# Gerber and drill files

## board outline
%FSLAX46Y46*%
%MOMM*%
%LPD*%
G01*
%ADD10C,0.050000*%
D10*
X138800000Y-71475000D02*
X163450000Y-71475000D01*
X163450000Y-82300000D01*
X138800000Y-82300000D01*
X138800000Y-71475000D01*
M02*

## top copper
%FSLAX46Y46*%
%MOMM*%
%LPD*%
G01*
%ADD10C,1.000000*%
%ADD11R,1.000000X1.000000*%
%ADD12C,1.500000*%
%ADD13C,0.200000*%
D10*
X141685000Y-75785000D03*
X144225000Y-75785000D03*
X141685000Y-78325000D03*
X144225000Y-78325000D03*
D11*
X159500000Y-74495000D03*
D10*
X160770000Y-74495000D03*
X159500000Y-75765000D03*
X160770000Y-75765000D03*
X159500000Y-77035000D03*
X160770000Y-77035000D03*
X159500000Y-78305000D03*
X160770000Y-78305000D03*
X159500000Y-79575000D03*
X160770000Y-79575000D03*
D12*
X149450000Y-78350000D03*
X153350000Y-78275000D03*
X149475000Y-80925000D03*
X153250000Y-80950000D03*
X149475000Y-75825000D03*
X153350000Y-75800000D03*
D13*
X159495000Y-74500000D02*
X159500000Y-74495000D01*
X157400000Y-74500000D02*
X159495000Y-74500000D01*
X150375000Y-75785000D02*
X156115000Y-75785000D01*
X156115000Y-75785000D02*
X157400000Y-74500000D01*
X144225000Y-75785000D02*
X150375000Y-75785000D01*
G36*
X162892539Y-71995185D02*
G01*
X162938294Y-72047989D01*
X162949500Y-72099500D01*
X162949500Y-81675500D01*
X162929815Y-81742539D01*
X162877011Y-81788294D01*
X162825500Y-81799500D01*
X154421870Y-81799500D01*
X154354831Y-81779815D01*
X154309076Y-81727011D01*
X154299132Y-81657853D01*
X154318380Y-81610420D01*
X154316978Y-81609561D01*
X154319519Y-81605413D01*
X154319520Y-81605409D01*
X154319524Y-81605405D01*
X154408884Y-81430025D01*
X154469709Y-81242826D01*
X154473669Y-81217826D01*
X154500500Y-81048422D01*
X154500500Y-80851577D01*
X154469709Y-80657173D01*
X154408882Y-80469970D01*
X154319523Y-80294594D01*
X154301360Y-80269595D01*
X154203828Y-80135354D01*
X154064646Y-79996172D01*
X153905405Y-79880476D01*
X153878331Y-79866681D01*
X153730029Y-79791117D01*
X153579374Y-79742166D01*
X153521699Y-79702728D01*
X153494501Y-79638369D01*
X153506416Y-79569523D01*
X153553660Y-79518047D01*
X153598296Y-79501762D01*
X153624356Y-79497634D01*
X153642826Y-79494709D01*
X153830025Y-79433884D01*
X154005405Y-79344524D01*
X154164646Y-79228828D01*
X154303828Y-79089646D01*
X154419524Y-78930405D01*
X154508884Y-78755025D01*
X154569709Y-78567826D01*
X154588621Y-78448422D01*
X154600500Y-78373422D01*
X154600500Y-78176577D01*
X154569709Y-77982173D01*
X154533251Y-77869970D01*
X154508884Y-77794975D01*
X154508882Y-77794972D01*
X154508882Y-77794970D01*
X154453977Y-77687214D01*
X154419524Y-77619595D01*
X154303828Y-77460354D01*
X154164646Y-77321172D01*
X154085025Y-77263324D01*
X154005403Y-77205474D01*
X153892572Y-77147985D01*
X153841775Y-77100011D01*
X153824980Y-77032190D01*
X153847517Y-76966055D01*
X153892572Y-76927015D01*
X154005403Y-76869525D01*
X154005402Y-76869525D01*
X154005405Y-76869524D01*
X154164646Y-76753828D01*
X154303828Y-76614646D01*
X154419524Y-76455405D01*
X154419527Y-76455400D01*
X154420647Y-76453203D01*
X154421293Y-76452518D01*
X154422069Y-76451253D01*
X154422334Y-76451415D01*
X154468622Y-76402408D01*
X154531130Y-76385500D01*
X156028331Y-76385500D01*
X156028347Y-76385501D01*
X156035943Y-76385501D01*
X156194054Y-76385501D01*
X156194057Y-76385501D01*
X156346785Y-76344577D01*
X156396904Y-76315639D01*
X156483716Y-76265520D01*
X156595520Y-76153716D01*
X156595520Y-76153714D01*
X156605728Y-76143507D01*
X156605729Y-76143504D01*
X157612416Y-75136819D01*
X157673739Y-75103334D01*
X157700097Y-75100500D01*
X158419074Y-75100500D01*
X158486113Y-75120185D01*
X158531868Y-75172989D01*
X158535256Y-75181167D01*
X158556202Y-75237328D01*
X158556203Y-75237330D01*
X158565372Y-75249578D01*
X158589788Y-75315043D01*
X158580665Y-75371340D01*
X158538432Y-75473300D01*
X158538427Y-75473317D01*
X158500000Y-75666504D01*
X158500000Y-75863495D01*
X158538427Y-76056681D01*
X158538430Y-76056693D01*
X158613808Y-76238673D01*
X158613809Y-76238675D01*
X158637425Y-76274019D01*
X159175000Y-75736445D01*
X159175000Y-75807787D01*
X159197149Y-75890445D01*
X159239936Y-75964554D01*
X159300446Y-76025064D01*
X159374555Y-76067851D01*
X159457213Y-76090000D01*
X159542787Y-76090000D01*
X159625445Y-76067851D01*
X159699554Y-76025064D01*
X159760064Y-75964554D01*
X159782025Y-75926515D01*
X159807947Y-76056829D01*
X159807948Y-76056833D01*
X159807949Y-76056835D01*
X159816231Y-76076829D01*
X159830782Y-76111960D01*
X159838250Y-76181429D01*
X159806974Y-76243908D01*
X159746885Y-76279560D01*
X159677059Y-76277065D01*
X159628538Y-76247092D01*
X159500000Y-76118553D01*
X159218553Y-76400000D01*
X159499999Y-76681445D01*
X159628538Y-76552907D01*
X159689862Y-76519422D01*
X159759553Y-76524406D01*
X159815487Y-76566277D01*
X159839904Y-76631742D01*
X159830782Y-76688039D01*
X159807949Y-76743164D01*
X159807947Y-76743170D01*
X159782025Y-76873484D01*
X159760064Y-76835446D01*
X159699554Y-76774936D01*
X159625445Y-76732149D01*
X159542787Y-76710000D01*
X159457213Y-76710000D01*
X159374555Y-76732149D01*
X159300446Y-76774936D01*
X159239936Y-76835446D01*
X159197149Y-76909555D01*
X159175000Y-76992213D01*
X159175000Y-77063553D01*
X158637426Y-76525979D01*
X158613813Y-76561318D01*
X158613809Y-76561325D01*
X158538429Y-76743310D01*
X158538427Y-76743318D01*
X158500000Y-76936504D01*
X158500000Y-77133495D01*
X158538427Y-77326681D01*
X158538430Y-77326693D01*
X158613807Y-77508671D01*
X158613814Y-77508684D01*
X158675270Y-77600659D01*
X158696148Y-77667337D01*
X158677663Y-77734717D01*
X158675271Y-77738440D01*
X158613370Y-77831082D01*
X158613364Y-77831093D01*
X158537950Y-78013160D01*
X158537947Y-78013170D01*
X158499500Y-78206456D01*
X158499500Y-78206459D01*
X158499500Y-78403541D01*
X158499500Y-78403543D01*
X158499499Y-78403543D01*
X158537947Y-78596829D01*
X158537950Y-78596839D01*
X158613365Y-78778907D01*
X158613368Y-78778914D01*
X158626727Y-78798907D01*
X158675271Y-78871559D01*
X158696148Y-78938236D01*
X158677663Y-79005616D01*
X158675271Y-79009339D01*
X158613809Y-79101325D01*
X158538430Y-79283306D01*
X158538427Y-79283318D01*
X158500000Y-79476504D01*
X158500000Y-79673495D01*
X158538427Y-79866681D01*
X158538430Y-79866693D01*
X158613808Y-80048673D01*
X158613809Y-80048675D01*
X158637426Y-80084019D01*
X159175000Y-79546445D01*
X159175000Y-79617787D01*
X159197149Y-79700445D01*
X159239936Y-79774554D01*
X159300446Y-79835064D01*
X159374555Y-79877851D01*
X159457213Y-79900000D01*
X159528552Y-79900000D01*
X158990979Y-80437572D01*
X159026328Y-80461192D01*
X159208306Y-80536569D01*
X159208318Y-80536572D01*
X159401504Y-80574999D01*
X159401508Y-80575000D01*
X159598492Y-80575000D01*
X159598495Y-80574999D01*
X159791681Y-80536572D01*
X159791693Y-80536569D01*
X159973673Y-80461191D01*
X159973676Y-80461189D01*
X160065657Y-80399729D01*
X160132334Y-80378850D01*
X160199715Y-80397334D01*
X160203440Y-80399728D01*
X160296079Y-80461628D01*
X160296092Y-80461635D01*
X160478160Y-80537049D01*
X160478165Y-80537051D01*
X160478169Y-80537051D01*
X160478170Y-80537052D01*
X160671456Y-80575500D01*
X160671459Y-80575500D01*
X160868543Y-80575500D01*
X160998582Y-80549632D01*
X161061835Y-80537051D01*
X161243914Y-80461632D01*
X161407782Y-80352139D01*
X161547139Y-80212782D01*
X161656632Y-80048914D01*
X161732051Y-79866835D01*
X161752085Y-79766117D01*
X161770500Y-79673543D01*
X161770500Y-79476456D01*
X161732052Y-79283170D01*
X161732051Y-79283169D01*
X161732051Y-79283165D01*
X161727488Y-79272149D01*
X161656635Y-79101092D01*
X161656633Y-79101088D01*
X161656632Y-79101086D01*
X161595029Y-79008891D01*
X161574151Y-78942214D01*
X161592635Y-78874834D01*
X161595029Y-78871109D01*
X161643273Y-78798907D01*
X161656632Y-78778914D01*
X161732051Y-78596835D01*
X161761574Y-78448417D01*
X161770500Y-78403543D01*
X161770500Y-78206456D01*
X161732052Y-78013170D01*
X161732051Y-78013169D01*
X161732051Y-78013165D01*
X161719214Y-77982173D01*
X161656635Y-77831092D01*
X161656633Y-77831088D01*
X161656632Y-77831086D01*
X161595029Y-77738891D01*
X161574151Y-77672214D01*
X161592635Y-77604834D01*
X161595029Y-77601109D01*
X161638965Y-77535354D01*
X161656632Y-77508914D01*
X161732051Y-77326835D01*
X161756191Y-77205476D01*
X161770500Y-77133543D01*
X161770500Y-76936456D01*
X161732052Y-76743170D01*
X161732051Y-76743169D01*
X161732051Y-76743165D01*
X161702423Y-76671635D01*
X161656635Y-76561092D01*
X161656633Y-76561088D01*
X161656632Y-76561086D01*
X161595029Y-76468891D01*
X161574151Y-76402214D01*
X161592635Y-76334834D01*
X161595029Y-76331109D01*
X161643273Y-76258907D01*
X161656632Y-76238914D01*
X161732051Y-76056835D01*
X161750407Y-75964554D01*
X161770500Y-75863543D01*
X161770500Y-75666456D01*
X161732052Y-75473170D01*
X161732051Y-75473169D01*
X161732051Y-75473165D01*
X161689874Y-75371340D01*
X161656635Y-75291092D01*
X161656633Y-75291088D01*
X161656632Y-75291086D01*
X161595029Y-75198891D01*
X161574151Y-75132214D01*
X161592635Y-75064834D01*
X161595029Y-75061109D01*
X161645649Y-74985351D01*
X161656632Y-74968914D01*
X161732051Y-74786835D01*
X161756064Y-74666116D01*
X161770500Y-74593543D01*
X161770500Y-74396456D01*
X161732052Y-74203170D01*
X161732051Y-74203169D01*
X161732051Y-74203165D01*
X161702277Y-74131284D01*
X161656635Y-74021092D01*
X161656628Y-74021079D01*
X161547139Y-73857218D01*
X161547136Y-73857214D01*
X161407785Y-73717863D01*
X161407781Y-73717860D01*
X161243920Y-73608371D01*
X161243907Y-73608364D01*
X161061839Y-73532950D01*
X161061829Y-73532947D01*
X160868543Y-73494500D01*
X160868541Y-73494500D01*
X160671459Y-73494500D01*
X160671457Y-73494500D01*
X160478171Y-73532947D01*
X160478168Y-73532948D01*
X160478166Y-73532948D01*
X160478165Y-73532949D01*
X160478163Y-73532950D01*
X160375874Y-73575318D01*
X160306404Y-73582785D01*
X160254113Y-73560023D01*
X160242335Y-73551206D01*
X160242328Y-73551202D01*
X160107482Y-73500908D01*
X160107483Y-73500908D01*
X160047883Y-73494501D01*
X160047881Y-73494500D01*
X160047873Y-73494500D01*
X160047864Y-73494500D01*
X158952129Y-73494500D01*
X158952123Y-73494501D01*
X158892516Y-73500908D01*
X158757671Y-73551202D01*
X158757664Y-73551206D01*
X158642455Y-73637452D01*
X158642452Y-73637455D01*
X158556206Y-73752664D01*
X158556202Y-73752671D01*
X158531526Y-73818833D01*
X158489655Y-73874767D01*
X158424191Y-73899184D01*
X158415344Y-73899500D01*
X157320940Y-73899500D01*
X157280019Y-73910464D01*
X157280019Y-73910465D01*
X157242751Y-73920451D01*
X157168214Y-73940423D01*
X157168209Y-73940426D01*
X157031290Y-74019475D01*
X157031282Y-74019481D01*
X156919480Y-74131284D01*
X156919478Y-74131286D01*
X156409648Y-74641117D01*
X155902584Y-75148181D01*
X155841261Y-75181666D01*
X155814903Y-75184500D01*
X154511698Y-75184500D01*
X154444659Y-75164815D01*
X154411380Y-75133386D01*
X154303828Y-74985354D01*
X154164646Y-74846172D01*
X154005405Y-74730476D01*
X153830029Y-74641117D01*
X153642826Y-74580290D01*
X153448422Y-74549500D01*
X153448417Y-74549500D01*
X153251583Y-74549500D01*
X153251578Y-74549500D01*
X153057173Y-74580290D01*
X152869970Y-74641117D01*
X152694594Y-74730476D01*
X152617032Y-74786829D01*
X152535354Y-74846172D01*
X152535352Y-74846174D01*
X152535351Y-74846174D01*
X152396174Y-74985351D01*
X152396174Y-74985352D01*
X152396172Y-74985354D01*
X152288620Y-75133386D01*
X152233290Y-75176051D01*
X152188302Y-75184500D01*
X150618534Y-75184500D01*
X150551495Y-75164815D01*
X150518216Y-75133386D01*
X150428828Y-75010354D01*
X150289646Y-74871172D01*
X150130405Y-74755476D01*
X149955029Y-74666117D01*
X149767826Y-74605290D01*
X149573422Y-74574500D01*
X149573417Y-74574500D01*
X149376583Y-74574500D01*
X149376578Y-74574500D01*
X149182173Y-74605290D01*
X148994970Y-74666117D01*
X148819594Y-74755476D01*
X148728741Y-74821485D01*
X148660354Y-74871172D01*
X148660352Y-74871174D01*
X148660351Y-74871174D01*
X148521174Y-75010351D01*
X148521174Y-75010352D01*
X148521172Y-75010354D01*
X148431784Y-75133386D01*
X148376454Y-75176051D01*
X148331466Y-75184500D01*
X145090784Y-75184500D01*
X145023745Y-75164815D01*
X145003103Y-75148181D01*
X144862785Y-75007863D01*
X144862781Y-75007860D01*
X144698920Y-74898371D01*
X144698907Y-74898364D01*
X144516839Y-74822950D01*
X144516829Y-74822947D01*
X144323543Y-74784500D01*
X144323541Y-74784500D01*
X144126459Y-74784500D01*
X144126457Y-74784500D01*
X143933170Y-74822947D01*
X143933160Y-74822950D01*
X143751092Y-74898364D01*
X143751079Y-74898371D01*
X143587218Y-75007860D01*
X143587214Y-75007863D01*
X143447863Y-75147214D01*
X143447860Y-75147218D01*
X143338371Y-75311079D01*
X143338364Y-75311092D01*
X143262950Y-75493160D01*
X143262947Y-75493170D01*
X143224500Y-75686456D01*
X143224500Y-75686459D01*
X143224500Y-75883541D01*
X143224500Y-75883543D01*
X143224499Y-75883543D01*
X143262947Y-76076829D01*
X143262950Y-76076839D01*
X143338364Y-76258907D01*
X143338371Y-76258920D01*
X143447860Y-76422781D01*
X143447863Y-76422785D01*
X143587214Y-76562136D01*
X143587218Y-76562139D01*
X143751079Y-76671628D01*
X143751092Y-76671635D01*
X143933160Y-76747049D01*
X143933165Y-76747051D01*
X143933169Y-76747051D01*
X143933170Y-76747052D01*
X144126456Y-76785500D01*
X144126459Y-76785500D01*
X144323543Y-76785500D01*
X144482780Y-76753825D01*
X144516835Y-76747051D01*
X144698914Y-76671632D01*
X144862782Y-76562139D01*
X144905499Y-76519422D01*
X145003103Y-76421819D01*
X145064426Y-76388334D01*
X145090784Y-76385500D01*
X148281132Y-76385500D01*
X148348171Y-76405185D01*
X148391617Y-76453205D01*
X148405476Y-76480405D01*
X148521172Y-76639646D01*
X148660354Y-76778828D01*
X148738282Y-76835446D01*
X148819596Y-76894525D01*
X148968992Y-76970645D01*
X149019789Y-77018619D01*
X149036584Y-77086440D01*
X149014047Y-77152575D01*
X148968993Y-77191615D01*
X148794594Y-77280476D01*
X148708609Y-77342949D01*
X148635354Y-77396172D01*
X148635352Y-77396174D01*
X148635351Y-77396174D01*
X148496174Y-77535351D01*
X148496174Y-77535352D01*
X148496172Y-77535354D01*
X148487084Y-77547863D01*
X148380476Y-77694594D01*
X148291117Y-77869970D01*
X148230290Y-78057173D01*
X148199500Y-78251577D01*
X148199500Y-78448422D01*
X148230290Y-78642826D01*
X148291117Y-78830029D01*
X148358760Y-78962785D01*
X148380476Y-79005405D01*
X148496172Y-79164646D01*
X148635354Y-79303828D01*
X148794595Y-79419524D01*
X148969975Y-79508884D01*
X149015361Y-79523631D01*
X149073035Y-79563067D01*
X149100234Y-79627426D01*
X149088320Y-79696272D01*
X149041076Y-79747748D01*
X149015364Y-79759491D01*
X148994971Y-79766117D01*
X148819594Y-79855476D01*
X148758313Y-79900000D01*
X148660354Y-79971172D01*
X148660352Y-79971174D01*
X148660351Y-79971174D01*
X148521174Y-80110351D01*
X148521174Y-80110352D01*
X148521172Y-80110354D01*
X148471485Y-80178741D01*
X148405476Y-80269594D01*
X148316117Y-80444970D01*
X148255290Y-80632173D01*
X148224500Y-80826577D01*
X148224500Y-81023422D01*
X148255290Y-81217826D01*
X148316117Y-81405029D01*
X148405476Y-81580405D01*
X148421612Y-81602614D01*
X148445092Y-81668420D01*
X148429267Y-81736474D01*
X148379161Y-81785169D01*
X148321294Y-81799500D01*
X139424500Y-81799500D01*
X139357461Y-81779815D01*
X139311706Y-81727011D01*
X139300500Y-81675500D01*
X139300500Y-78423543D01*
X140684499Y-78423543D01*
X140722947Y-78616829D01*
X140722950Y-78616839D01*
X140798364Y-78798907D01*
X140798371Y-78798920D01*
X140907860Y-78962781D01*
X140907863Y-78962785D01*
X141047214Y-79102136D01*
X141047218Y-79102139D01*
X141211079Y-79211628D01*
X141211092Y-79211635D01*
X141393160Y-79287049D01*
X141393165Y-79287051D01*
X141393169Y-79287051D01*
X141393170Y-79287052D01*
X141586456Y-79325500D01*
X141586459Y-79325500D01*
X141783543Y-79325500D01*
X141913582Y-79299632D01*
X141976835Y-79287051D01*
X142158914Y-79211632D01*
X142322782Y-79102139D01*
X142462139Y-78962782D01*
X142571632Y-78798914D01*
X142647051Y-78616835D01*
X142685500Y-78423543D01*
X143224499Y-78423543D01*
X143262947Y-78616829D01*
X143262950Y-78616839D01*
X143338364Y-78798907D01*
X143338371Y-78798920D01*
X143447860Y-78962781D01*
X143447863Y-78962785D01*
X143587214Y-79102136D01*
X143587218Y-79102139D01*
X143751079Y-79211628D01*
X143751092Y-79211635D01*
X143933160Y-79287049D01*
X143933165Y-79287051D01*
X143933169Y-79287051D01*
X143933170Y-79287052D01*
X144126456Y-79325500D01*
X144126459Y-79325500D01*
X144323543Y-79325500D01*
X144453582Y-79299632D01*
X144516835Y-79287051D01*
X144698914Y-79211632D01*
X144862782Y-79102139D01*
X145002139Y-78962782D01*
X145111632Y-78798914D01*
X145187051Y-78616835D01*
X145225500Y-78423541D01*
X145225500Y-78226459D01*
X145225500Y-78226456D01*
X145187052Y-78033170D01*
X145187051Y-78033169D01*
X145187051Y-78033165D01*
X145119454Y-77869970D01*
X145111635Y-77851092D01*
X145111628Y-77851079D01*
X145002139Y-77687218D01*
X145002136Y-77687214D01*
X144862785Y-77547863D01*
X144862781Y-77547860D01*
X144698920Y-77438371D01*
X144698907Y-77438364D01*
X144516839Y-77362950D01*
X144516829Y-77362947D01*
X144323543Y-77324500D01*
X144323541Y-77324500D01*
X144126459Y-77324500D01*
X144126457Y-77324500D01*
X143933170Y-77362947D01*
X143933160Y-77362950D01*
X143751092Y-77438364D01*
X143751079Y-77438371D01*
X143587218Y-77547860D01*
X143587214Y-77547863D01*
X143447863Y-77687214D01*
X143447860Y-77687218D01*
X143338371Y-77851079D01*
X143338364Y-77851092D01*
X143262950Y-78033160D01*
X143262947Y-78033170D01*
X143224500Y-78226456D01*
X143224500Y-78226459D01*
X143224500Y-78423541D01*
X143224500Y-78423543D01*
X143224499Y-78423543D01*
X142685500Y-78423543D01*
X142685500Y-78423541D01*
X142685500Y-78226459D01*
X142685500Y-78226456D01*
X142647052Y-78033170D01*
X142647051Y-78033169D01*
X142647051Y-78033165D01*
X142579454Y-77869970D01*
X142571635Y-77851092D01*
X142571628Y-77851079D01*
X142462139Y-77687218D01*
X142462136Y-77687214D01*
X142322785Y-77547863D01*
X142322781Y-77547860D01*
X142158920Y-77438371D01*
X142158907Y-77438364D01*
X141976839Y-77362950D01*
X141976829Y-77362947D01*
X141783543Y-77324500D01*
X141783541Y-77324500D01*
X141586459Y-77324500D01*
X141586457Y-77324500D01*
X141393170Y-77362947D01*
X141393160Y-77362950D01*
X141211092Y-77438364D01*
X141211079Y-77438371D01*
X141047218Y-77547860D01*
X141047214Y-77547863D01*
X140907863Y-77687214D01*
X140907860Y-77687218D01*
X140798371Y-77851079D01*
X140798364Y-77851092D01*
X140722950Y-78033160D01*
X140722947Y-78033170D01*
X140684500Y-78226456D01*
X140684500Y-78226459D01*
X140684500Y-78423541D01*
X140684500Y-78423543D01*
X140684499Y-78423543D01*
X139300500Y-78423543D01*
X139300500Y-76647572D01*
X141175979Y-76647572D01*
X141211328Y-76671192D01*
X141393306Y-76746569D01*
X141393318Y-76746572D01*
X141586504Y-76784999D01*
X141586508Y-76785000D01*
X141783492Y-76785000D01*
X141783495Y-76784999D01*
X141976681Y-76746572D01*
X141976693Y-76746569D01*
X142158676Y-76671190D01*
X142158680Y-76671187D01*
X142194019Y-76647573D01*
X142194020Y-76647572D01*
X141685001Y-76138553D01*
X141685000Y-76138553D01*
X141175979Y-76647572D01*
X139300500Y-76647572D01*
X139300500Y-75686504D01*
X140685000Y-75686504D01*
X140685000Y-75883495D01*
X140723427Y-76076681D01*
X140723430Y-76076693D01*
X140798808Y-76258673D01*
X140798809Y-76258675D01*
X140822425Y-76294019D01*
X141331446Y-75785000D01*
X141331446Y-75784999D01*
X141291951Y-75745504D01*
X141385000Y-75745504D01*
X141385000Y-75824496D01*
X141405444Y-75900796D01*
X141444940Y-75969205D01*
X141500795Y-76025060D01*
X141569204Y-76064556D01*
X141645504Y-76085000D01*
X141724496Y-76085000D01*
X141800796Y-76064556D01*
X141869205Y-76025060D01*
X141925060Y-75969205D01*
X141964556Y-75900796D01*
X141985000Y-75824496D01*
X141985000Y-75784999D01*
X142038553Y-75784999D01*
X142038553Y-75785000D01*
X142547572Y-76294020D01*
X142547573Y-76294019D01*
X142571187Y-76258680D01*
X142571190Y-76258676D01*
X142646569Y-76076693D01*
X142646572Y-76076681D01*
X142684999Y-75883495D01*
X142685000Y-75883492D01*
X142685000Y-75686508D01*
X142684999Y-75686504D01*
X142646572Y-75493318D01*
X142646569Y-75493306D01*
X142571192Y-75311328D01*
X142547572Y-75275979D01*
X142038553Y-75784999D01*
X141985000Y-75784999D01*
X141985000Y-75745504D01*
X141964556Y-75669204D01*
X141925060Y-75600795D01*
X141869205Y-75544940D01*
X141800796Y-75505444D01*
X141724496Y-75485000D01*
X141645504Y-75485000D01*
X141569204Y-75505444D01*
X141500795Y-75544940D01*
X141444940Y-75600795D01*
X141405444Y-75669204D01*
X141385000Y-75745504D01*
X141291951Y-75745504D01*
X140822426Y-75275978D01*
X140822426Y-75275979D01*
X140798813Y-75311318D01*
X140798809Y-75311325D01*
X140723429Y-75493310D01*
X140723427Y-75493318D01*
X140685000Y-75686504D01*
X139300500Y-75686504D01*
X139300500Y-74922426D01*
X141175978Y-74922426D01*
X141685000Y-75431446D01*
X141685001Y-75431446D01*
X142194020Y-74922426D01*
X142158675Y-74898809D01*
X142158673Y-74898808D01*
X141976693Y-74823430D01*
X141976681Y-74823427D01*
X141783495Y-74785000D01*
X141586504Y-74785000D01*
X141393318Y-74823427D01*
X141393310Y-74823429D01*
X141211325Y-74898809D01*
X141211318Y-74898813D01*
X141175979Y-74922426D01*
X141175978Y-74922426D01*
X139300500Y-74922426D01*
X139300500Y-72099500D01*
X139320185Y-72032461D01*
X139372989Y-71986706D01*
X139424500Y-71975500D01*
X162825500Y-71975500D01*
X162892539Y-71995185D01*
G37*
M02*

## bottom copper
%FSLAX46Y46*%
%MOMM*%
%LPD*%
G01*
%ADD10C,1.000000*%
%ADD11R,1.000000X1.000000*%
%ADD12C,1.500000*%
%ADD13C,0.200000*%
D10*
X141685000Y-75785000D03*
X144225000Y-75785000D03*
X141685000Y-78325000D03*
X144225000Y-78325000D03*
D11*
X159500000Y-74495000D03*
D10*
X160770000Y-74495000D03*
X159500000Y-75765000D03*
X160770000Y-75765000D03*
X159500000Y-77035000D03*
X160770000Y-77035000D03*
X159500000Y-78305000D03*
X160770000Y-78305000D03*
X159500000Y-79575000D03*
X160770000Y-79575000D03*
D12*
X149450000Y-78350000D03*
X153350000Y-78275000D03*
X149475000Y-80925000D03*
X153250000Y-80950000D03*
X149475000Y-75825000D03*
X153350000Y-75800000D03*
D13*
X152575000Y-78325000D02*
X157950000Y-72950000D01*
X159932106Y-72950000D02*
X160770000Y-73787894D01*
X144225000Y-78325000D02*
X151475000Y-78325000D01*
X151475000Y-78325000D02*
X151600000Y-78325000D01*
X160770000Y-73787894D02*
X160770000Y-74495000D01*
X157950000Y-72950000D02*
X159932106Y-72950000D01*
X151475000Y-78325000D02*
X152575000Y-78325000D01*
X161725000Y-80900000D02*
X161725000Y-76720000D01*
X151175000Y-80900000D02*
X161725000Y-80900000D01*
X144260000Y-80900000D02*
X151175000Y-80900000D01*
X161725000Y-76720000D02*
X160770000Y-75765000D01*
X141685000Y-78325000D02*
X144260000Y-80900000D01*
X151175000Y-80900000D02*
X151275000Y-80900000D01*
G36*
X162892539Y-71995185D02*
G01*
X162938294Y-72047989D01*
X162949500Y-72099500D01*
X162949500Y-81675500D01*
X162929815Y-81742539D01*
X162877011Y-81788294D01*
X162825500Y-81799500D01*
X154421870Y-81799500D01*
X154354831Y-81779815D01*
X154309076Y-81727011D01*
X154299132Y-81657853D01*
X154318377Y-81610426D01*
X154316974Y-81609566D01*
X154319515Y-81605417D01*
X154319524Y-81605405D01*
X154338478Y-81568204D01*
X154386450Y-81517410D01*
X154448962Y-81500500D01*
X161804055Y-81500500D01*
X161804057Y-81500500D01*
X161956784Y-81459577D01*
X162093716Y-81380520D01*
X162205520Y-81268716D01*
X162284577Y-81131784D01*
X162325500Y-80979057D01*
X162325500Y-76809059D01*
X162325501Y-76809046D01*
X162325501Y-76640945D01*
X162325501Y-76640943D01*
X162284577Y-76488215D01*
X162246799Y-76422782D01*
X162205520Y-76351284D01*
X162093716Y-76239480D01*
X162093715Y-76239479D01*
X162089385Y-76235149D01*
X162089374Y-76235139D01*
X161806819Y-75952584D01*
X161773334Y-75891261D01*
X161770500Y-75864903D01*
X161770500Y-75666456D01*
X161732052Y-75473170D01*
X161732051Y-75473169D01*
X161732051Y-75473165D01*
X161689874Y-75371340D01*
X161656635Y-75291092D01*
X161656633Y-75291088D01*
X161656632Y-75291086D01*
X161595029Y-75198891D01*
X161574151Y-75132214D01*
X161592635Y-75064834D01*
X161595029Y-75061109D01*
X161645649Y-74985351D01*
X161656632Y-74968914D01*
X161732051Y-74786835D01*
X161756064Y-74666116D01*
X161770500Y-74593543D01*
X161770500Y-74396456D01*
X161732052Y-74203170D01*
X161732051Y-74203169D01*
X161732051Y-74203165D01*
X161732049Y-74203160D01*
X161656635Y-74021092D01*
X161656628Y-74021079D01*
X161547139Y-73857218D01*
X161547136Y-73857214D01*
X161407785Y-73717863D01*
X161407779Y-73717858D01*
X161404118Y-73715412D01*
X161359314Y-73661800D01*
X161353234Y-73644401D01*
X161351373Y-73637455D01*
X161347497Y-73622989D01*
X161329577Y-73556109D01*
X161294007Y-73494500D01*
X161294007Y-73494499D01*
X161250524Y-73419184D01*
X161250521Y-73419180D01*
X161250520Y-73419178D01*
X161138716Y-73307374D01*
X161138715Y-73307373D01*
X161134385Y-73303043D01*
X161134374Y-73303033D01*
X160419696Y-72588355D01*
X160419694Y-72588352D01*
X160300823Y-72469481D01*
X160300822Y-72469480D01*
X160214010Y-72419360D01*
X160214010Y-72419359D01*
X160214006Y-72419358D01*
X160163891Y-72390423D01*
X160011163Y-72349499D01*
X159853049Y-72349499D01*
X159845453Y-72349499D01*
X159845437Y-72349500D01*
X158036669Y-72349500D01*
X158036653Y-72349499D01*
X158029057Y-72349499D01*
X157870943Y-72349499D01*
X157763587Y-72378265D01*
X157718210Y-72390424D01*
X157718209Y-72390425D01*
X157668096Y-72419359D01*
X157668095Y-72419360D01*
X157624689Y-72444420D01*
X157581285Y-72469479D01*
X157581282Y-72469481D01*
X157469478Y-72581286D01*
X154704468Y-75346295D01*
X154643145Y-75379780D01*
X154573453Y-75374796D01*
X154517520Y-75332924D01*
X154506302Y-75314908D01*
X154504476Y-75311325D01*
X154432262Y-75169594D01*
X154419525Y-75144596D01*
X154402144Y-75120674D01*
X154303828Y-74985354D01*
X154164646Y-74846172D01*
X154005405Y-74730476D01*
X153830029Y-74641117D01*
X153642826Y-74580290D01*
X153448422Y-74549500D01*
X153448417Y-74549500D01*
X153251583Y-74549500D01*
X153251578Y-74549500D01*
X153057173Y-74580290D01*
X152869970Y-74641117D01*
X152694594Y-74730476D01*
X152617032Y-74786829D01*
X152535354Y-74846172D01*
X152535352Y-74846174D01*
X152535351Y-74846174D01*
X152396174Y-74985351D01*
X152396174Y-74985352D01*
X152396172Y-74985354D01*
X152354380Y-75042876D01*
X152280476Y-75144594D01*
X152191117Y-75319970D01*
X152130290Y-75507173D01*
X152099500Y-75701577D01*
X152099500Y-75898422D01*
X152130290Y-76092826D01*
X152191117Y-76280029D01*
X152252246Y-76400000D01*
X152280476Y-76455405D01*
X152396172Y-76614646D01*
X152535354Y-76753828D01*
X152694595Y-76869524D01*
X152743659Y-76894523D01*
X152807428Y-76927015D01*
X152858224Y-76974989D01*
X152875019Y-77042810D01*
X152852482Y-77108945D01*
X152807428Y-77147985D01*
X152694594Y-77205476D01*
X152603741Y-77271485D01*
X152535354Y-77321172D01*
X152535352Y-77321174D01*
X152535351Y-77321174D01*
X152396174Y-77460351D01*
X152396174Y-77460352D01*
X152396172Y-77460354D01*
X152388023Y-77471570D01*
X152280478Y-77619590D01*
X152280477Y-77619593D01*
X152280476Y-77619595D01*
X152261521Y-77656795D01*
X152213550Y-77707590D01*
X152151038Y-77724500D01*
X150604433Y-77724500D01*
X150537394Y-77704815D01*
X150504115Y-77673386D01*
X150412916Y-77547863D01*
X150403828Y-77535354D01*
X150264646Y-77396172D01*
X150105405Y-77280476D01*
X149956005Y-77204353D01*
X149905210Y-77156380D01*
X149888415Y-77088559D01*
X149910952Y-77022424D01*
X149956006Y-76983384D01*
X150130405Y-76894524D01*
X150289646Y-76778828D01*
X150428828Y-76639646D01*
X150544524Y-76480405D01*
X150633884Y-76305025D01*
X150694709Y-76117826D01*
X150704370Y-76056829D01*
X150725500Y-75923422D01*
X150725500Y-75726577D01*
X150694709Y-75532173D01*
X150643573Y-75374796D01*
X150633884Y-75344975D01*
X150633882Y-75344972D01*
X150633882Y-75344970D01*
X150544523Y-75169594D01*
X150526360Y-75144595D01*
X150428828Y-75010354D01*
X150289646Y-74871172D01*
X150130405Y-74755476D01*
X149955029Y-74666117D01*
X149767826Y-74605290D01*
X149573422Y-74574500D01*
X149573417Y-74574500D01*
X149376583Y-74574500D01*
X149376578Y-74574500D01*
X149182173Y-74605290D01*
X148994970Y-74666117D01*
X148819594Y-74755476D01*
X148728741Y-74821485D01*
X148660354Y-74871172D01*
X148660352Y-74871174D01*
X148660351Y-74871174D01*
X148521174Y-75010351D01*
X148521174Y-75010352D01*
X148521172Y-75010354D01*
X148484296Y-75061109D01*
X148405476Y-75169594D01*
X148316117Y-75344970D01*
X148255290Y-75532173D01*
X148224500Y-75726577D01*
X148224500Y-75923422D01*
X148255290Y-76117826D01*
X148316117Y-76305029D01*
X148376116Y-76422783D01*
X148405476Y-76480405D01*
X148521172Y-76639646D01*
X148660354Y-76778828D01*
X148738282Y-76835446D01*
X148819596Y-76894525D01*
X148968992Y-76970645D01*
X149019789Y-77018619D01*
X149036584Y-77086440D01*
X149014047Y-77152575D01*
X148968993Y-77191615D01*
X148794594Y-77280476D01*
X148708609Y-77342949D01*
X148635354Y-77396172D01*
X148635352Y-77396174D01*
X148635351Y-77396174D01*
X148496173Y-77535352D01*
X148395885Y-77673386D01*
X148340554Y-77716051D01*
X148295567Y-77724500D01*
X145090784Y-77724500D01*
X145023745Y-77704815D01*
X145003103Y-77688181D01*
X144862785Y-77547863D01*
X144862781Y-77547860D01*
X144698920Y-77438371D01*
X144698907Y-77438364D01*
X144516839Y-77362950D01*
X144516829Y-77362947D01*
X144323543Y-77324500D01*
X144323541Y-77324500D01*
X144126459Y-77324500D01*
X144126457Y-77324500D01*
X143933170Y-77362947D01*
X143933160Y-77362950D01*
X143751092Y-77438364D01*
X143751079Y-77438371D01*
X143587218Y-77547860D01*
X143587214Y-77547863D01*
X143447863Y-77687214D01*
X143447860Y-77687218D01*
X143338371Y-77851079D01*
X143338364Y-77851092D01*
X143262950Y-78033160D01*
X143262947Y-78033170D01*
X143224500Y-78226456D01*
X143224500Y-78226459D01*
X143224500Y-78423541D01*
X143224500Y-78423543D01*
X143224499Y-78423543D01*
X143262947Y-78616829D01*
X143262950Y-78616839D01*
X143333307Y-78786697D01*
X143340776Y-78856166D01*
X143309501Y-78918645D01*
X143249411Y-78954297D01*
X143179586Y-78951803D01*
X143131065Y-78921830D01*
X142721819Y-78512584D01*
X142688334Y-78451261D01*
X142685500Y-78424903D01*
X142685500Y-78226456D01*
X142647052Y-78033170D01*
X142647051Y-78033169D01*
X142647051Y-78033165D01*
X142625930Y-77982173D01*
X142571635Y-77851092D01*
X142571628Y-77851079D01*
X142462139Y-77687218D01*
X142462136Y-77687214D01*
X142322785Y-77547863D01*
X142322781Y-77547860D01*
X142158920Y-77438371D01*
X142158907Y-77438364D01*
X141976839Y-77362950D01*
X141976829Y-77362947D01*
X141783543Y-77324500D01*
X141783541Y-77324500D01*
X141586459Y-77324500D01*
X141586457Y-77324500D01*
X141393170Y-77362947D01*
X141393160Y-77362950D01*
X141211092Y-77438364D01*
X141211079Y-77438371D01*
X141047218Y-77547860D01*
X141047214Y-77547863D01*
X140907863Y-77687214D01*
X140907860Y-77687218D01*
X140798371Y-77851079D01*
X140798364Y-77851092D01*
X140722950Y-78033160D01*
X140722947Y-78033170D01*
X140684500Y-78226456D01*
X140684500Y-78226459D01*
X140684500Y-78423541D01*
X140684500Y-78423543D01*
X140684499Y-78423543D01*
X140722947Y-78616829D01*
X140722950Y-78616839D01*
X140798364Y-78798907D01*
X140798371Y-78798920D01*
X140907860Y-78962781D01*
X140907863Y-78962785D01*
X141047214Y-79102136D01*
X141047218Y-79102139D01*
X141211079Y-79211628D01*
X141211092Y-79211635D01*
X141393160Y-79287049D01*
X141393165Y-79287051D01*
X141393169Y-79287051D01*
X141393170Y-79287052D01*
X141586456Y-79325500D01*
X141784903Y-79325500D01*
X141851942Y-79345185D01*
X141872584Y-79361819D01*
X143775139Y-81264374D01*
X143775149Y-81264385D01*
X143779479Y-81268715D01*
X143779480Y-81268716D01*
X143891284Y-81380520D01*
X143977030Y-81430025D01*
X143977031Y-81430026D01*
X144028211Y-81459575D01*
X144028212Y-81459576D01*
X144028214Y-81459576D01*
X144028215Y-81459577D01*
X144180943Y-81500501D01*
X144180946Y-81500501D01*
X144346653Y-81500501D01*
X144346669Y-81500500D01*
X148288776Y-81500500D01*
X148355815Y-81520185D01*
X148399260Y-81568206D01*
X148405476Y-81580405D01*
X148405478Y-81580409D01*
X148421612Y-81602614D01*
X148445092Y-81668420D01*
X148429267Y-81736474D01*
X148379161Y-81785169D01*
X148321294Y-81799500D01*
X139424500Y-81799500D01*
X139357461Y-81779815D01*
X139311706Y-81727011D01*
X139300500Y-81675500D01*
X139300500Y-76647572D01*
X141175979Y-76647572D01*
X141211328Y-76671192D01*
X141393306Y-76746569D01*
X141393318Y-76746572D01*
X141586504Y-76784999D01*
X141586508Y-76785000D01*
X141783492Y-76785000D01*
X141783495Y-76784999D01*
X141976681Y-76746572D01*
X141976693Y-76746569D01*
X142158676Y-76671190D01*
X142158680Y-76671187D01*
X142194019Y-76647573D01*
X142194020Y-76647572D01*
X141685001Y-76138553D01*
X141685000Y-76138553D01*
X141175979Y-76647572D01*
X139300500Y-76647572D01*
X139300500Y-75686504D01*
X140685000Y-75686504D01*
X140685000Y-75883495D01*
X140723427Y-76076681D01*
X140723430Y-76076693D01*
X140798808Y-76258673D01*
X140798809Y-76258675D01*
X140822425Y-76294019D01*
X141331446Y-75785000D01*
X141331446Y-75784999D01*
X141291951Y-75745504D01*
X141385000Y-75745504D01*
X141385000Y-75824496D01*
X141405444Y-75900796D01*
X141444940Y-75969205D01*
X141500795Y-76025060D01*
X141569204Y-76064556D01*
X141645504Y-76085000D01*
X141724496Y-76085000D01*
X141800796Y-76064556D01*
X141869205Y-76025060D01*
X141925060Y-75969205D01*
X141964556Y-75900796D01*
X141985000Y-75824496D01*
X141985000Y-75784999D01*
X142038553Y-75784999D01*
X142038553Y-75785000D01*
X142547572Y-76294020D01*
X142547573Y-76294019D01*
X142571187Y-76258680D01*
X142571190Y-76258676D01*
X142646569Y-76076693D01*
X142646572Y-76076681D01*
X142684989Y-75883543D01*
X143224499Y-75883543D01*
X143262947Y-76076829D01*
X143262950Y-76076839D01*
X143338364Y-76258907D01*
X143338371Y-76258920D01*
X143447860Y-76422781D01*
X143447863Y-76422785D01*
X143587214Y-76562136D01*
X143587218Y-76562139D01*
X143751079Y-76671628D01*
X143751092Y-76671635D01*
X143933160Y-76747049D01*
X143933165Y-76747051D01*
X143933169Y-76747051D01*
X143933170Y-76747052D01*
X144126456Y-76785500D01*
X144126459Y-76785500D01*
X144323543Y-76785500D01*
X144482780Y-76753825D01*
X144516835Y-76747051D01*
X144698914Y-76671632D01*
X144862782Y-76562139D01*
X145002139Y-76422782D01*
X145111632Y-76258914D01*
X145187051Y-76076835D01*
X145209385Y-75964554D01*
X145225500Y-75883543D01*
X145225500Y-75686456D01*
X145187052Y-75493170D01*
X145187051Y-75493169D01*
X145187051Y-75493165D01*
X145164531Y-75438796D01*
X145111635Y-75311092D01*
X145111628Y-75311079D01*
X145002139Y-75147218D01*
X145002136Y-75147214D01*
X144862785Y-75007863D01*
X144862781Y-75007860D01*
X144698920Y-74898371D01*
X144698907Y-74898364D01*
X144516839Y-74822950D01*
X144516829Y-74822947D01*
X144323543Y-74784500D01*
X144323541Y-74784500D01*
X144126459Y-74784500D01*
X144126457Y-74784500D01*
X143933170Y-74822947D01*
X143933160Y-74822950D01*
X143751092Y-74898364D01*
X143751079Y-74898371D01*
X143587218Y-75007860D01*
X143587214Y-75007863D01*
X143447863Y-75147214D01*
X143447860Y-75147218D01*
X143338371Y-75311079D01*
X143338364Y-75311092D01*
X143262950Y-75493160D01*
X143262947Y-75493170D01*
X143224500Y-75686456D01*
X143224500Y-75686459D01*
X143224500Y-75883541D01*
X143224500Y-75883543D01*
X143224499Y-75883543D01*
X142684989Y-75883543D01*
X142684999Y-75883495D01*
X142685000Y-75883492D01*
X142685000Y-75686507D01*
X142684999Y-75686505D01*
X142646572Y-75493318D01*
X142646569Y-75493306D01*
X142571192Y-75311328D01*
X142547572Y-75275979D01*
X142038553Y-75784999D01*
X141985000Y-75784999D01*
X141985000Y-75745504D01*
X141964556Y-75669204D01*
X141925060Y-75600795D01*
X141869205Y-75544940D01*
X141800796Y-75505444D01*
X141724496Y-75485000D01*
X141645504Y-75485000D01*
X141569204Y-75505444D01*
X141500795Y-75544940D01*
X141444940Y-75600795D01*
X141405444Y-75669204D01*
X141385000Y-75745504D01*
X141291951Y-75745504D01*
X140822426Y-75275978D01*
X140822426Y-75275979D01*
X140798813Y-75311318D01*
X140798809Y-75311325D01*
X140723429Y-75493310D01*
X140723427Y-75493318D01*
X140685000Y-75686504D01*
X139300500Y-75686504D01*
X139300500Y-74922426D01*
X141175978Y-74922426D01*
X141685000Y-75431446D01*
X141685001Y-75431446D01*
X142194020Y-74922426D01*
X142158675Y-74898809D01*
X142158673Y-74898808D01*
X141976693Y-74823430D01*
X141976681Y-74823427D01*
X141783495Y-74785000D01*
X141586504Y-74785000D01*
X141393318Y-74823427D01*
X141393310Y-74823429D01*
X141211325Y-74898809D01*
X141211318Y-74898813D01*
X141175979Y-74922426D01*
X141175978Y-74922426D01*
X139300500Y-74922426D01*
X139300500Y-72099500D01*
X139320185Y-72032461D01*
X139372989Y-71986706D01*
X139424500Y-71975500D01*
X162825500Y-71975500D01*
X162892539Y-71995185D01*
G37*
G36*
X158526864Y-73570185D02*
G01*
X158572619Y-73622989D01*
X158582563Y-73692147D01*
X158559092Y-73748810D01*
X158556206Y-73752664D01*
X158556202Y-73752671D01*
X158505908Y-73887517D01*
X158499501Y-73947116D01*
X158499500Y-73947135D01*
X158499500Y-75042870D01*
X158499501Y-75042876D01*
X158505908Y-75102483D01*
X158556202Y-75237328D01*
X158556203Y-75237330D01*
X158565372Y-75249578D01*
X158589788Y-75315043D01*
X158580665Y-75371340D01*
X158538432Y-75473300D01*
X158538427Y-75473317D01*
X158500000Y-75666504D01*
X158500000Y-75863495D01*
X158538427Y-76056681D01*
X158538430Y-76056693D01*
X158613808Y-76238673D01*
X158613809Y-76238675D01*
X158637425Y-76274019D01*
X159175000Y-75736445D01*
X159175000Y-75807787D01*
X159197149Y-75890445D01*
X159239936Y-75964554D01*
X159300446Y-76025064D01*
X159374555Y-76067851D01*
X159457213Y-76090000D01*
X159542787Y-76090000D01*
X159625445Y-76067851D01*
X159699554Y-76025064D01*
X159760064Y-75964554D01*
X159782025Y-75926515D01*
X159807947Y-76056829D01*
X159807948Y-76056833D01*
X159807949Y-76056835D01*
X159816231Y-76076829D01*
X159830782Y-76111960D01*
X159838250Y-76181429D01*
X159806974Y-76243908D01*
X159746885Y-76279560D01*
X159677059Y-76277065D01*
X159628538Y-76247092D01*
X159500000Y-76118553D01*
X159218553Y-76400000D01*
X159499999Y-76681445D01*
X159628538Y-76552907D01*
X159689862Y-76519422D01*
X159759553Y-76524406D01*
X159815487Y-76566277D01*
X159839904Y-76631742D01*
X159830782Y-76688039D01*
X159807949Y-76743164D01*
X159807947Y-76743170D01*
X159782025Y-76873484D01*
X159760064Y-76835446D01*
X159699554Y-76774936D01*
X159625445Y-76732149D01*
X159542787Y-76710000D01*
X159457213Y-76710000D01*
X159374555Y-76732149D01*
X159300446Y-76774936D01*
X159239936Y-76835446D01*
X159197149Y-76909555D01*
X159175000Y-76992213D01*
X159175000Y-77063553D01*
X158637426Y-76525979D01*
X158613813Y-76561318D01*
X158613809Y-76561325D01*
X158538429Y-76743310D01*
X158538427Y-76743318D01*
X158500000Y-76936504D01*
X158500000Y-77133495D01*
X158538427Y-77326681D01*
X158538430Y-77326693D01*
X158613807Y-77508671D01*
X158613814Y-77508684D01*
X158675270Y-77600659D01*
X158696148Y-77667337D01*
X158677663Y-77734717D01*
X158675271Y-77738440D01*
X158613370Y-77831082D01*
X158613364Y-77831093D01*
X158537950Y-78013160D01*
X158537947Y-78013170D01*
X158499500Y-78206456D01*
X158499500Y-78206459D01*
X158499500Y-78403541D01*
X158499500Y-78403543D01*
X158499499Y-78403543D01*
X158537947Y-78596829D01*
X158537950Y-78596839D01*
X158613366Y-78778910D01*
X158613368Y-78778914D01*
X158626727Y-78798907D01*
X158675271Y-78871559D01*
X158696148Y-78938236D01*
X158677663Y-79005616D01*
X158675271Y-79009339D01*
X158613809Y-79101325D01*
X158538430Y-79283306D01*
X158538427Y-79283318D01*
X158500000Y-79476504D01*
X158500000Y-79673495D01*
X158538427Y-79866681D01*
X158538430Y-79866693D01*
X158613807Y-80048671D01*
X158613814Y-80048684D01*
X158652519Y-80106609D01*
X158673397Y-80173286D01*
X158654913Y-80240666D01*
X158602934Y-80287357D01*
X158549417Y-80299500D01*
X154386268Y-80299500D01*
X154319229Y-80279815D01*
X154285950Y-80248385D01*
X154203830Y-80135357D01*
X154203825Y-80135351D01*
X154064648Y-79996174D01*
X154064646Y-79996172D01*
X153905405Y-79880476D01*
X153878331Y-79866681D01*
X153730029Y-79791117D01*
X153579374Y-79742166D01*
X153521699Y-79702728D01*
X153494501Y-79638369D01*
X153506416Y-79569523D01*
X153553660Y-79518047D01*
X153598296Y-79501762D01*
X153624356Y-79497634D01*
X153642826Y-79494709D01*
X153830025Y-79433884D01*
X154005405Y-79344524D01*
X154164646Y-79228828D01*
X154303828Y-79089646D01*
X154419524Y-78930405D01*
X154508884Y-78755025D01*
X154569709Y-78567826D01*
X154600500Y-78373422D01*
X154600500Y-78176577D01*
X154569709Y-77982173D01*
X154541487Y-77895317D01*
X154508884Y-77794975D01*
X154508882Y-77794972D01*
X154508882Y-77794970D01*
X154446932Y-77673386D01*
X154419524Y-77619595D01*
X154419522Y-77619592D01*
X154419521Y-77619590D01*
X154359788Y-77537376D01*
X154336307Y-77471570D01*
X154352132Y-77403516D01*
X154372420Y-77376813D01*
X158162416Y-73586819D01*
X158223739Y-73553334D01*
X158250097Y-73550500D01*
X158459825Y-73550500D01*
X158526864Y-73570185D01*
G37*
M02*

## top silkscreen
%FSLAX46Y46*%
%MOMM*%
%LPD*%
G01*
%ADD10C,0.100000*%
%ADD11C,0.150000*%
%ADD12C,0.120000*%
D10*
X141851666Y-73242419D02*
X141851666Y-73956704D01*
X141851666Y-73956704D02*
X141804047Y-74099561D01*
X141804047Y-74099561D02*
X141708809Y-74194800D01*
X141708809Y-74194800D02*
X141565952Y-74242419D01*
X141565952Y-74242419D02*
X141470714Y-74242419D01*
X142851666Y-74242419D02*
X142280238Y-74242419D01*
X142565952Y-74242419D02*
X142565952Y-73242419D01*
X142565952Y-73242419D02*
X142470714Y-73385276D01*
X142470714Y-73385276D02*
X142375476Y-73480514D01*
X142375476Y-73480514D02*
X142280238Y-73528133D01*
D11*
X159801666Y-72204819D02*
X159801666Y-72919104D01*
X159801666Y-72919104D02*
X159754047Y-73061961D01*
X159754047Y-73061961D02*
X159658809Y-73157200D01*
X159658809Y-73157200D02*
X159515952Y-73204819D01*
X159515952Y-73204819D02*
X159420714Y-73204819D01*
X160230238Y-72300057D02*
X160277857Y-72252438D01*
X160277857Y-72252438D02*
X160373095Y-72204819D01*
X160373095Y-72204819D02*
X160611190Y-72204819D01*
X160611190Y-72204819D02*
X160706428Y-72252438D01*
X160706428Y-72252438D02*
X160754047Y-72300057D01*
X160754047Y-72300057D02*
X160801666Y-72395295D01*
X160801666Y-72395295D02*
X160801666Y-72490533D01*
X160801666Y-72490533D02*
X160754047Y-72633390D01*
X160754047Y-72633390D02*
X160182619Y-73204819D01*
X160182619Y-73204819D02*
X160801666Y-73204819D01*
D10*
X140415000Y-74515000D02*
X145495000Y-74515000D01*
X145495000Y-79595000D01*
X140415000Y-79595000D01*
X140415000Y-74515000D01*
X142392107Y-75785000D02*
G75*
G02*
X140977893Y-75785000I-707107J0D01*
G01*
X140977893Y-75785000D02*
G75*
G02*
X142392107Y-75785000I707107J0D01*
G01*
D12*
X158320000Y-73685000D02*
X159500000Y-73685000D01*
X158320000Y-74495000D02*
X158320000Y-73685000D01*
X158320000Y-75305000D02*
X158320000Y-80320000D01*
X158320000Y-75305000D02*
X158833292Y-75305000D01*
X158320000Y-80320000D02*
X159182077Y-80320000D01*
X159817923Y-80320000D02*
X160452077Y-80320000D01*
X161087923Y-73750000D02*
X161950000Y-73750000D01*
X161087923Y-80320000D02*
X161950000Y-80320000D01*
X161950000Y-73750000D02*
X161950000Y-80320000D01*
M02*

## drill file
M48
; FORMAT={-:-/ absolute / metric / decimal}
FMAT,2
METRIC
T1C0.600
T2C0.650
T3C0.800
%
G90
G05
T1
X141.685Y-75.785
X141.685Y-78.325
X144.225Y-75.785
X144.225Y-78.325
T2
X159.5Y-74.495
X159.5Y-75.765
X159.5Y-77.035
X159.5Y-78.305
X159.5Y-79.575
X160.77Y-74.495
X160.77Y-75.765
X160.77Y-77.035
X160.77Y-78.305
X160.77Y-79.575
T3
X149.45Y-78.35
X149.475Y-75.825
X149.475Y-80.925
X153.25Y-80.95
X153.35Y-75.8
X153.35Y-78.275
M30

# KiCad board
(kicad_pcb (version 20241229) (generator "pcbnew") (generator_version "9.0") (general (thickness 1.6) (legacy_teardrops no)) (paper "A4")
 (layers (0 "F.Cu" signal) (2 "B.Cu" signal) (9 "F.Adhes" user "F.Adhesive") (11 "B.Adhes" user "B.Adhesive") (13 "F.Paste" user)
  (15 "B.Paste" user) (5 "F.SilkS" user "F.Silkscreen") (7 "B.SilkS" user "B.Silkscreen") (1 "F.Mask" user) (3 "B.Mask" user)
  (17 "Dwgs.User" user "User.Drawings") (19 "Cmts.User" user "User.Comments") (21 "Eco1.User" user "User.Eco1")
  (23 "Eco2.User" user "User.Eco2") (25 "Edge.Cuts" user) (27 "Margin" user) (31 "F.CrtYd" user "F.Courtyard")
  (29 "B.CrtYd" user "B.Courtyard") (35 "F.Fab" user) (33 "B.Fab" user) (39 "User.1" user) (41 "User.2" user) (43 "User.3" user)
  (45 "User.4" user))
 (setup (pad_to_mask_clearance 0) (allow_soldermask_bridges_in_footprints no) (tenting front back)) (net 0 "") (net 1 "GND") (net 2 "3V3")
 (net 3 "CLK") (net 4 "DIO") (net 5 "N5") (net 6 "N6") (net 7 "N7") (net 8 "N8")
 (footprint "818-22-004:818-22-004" (layer "F.Cu") (at 141.685 75.785)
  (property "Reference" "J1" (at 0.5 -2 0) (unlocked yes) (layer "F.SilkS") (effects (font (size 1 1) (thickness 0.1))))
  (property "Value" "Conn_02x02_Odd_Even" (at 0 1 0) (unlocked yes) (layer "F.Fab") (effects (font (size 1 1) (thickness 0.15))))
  (fp_rect (start -1.27 -1.27) (end 3.81 3.81) (stroke (width 0.1) (type solid)) (fill no) (layer "F.SilkS"))
  (fp_circle (center 0 0) (end 0.5 0.5) (stroke (width 0.1) (type default)) (fill no) (layer "F.SilkS"))
  (pad "1" thru_hole circle (at 0 0) (size 1 1) (drill 0.6) (layers "*.Cu" "*.Mask") (remove_unused_layers no) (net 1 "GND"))
  (pad "2" thru_hole circle (at 2.54 0) (size 1 1) (drill 0.6) (layers "*.Cu" "*.Mask") (remove_unused_layers no) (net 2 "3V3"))
  (pad "3" thru_hole circle (at 0 2.54) (size 1 1) (drill 0.6) (layers "*.Cu" "*.Mask") (remove_unused_layers no) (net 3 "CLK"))
  (pad "4" thru_hole circle (at 2.54 2.54) (size 1 1) (drill 0.6) (layers "*.Cu" "*.Mask") (remove_unused_layers no) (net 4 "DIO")))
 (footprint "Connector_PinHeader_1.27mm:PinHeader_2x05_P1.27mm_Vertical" (layer "F.Cu") (at 159.5 74.495)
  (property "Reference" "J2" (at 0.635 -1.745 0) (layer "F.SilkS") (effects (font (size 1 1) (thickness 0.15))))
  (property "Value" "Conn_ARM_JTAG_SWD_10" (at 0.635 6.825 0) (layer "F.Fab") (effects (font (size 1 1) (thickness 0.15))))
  (fp_line (start -1.18 -0.81) (end 0 -0.81) (stroke (width 0.12) (type solid)) (layer "F.SilkS"))
  (fp_line (start -1.18 0) (end -1.18 -0.81) (stroke (width 0.12) (type solid)) (layer "F.SilkS"))
  (fp_line (start -1.18 0.81) (end -1.18 5.825) (stroke (width 0.12) (type solid)) (layer "F.SilkS"))
  (fp_line (start -1.18 0.81) (end -0.666708 0.81) (stroke (width 0.12) (type solid)) (layer "F.SilkS"))
  (fp_line (start -1.18 5.825) (end -0.317923 5.825) (stroke (width 0.12) (type solid)) (layer "F.SilkS"))
  (fp_line (start 0.317923 5.825) (end 0.952077 5.825) (stroke (width 0.12) (type solid)) (layer "F.SilkS"))
  (fp_line (start 1.587923 -0.745) (end 2.45 -0.745) (stroke (width 0.12) (type solid)) (layer "F.SilkS"))
  (fp_line (start 1.587923 5.825) (end 2.45 5.825) (stroke (width 0.12) (type solid)) (layer "F.SilkS"))
  (fp_line (start 2.45 -0.745) (end 2.45 5.825) (stroke (width 0.12) (type solid)) (layer "F.SilkS"))
  (pad "1" thru_hole rect (at 0 0) (size 1 1) (drill 0.65) (layers "*.Cu" "*.Mask") (remove_unused_layers no) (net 2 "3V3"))
  (pad "2" thru_hole circle (at 1.27 0) (size 1 1) (drill 0.65) (layers "*.Cu" "*.Mask") (remove_unused_layers no) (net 4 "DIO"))
  (pad "3" thru_hole circle (at 0 1.27) (size 1 1) (drill 0.65) (layers "*.Cu" "*.Mask") (remove_unused_layers no) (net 1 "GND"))
  (pad "4" thru_hole circle (at 1.27 1.27) (size 1 1) (drill 0.65) (layers "*.Cu" "*.Mask") (remove_unused_layers no) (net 3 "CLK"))
  (pad "5" thru_hole circle (at 0 2.54) (size 1 1) (drill 0.65) (layers "*.Cu" "*.Mask") (remove_unused_layers no) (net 1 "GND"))
  (pad "6" thru_hole circle (at 1.27 2.54) (size 1 1) (drill 0.65) (layers "*.Cu" "*.Mask") (remove_unused_layers no) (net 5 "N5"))
  (pad "7" thru_hole circle (at 0 3.81) (size 1 1) (drill 0.65) (layers "*.Cu" "*.Mask") (remove_unused_layers no) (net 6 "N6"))
  (pad "8" thru_hole circle (at 1.27 3.81) (size 1 1) (drill 0.65) (layers "*.Cu" "*.Mask") (remove_unused_layers no) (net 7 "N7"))
  (pad "9" thru_hole circle (at 0 5.08) (size 1 1) (drill 0.65) (layers "*.Cu" "*.Mask") (remove_unused_layers no) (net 1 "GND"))
  (pad "10" thru_hole circle (at 1.27 5.08) (size 1 1) (drill 0.65) (layers "*.Cu" "*.Mask") (remove_unused_layers no) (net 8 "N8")))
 (gr_rect (start 138.8 71.475) (end 163.45 82.3) (stroke (width 0.05) (type default)) (fill no) (layer "Edge.Cuts"))
 (via (at 149.45 78.35) (size 1.5) (drill 0.8) (layers "F.Cu" "B.Cu") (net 4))
 (via (at 153.35 78.275) (size 1.5) (drill 0.8) (layers "F.Cu" "B.Cu") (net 4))
 (segment (start 152.575 78.325) (end 157.95 72.95) (width 0.2) (layer "B.Cu") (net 4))
 (segment (start 159.932106 72.95) (end 160.77 73.787894) (width 0.2) (layer "B.Cu") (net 4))
 (segment (start 144.225 78.325) (end 151.475 78.325) (width 0.2) (layer "B.Cu") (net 4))
 (segment (start 151.475 78.325) (end 151.6 78.325) (width 0.2) (layer "B.Cu") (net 4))
 (segment (start 160.77 73.787894) (end 160.77 74.495) (width 0.2) (layer "B.Cu") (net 4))
 (segment (start 157.95 72.95) (end 159.932106 72.95) (width 0.2) (layer "B.Cu") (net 4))
 (segment (start 151.475 78.325) (end 152.575 78.325) (width 0.2) (layer "B.Cu") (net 4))
 (via (at 149.475 80.925) (size 1.5) (drill 0.8) (layers "F.Cu" "B.Cu") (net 3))
 (via (at 153.25 80.95) (size 1.5) (drill 0.8) (layers "F.Cu" "B.Cu") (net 3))
 (segment (start 161.725 80.9) (end 161.725 76.72) (width 0.2) (layer "B.Cu") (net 3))
 (segment (start 151.175 80.9) (end 161.725 80.9) (width 0.2) (layer "B.Cu") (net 3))
 (segment (start 144.26 80.9) (end 151.175 80.9) (width 0.2) (layer "B.Cu") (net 3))
 (segment (start 161.725 76.72) (end 160.77 75.765) (width 0.2) (layer "B.Cu") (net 3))
 (segment (start 141.685 78.325) (end 144.26 80.9) (width 0.2) (layer "B.Cu") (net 3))
 (segment (start 151.175 80.9) (end 151.275 80.9) (width 0.2) (layer "B.Cu") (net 3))
 (segment (start 159.495 74.5) (end 159.5 74.495) (width 0.2) (layer "F.Cu") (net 2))
 (segment (start 157.4 74.5) (end 159.495 74.5) (width 0.2) (layer "F.Cu") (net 2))
 (segment (start 150.375 75.785) (end 156.115 75.785) (width 0.2) (layer "F.Cu") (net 2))
 (segment (start 156.115 75.785) (end 157.4 74.5) (width 0.2) (layer "F.Cu") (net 2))
 (segment (start 144.225 75.785) (end 150.375 75.785) (width 0.2) (layer "F.Cu") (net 2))
 (via (at 149.475 75.825) (size 1.5) (drill 0.8) (layers "F.Cu" "B.Cu") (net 2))
 (via (at 153.35 75.8) (size 1.5) (drill 0.8) (layers "F.Cu" "B.Cu") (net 2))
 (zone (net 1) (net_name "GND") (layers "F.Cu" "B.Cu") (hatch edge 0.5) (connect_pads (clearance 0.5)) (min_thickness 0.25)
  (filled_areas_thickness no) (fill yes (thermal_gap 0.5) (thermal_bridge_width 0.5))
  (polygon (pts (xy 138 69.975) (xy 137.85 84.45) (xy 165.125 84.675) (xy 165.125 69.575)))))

